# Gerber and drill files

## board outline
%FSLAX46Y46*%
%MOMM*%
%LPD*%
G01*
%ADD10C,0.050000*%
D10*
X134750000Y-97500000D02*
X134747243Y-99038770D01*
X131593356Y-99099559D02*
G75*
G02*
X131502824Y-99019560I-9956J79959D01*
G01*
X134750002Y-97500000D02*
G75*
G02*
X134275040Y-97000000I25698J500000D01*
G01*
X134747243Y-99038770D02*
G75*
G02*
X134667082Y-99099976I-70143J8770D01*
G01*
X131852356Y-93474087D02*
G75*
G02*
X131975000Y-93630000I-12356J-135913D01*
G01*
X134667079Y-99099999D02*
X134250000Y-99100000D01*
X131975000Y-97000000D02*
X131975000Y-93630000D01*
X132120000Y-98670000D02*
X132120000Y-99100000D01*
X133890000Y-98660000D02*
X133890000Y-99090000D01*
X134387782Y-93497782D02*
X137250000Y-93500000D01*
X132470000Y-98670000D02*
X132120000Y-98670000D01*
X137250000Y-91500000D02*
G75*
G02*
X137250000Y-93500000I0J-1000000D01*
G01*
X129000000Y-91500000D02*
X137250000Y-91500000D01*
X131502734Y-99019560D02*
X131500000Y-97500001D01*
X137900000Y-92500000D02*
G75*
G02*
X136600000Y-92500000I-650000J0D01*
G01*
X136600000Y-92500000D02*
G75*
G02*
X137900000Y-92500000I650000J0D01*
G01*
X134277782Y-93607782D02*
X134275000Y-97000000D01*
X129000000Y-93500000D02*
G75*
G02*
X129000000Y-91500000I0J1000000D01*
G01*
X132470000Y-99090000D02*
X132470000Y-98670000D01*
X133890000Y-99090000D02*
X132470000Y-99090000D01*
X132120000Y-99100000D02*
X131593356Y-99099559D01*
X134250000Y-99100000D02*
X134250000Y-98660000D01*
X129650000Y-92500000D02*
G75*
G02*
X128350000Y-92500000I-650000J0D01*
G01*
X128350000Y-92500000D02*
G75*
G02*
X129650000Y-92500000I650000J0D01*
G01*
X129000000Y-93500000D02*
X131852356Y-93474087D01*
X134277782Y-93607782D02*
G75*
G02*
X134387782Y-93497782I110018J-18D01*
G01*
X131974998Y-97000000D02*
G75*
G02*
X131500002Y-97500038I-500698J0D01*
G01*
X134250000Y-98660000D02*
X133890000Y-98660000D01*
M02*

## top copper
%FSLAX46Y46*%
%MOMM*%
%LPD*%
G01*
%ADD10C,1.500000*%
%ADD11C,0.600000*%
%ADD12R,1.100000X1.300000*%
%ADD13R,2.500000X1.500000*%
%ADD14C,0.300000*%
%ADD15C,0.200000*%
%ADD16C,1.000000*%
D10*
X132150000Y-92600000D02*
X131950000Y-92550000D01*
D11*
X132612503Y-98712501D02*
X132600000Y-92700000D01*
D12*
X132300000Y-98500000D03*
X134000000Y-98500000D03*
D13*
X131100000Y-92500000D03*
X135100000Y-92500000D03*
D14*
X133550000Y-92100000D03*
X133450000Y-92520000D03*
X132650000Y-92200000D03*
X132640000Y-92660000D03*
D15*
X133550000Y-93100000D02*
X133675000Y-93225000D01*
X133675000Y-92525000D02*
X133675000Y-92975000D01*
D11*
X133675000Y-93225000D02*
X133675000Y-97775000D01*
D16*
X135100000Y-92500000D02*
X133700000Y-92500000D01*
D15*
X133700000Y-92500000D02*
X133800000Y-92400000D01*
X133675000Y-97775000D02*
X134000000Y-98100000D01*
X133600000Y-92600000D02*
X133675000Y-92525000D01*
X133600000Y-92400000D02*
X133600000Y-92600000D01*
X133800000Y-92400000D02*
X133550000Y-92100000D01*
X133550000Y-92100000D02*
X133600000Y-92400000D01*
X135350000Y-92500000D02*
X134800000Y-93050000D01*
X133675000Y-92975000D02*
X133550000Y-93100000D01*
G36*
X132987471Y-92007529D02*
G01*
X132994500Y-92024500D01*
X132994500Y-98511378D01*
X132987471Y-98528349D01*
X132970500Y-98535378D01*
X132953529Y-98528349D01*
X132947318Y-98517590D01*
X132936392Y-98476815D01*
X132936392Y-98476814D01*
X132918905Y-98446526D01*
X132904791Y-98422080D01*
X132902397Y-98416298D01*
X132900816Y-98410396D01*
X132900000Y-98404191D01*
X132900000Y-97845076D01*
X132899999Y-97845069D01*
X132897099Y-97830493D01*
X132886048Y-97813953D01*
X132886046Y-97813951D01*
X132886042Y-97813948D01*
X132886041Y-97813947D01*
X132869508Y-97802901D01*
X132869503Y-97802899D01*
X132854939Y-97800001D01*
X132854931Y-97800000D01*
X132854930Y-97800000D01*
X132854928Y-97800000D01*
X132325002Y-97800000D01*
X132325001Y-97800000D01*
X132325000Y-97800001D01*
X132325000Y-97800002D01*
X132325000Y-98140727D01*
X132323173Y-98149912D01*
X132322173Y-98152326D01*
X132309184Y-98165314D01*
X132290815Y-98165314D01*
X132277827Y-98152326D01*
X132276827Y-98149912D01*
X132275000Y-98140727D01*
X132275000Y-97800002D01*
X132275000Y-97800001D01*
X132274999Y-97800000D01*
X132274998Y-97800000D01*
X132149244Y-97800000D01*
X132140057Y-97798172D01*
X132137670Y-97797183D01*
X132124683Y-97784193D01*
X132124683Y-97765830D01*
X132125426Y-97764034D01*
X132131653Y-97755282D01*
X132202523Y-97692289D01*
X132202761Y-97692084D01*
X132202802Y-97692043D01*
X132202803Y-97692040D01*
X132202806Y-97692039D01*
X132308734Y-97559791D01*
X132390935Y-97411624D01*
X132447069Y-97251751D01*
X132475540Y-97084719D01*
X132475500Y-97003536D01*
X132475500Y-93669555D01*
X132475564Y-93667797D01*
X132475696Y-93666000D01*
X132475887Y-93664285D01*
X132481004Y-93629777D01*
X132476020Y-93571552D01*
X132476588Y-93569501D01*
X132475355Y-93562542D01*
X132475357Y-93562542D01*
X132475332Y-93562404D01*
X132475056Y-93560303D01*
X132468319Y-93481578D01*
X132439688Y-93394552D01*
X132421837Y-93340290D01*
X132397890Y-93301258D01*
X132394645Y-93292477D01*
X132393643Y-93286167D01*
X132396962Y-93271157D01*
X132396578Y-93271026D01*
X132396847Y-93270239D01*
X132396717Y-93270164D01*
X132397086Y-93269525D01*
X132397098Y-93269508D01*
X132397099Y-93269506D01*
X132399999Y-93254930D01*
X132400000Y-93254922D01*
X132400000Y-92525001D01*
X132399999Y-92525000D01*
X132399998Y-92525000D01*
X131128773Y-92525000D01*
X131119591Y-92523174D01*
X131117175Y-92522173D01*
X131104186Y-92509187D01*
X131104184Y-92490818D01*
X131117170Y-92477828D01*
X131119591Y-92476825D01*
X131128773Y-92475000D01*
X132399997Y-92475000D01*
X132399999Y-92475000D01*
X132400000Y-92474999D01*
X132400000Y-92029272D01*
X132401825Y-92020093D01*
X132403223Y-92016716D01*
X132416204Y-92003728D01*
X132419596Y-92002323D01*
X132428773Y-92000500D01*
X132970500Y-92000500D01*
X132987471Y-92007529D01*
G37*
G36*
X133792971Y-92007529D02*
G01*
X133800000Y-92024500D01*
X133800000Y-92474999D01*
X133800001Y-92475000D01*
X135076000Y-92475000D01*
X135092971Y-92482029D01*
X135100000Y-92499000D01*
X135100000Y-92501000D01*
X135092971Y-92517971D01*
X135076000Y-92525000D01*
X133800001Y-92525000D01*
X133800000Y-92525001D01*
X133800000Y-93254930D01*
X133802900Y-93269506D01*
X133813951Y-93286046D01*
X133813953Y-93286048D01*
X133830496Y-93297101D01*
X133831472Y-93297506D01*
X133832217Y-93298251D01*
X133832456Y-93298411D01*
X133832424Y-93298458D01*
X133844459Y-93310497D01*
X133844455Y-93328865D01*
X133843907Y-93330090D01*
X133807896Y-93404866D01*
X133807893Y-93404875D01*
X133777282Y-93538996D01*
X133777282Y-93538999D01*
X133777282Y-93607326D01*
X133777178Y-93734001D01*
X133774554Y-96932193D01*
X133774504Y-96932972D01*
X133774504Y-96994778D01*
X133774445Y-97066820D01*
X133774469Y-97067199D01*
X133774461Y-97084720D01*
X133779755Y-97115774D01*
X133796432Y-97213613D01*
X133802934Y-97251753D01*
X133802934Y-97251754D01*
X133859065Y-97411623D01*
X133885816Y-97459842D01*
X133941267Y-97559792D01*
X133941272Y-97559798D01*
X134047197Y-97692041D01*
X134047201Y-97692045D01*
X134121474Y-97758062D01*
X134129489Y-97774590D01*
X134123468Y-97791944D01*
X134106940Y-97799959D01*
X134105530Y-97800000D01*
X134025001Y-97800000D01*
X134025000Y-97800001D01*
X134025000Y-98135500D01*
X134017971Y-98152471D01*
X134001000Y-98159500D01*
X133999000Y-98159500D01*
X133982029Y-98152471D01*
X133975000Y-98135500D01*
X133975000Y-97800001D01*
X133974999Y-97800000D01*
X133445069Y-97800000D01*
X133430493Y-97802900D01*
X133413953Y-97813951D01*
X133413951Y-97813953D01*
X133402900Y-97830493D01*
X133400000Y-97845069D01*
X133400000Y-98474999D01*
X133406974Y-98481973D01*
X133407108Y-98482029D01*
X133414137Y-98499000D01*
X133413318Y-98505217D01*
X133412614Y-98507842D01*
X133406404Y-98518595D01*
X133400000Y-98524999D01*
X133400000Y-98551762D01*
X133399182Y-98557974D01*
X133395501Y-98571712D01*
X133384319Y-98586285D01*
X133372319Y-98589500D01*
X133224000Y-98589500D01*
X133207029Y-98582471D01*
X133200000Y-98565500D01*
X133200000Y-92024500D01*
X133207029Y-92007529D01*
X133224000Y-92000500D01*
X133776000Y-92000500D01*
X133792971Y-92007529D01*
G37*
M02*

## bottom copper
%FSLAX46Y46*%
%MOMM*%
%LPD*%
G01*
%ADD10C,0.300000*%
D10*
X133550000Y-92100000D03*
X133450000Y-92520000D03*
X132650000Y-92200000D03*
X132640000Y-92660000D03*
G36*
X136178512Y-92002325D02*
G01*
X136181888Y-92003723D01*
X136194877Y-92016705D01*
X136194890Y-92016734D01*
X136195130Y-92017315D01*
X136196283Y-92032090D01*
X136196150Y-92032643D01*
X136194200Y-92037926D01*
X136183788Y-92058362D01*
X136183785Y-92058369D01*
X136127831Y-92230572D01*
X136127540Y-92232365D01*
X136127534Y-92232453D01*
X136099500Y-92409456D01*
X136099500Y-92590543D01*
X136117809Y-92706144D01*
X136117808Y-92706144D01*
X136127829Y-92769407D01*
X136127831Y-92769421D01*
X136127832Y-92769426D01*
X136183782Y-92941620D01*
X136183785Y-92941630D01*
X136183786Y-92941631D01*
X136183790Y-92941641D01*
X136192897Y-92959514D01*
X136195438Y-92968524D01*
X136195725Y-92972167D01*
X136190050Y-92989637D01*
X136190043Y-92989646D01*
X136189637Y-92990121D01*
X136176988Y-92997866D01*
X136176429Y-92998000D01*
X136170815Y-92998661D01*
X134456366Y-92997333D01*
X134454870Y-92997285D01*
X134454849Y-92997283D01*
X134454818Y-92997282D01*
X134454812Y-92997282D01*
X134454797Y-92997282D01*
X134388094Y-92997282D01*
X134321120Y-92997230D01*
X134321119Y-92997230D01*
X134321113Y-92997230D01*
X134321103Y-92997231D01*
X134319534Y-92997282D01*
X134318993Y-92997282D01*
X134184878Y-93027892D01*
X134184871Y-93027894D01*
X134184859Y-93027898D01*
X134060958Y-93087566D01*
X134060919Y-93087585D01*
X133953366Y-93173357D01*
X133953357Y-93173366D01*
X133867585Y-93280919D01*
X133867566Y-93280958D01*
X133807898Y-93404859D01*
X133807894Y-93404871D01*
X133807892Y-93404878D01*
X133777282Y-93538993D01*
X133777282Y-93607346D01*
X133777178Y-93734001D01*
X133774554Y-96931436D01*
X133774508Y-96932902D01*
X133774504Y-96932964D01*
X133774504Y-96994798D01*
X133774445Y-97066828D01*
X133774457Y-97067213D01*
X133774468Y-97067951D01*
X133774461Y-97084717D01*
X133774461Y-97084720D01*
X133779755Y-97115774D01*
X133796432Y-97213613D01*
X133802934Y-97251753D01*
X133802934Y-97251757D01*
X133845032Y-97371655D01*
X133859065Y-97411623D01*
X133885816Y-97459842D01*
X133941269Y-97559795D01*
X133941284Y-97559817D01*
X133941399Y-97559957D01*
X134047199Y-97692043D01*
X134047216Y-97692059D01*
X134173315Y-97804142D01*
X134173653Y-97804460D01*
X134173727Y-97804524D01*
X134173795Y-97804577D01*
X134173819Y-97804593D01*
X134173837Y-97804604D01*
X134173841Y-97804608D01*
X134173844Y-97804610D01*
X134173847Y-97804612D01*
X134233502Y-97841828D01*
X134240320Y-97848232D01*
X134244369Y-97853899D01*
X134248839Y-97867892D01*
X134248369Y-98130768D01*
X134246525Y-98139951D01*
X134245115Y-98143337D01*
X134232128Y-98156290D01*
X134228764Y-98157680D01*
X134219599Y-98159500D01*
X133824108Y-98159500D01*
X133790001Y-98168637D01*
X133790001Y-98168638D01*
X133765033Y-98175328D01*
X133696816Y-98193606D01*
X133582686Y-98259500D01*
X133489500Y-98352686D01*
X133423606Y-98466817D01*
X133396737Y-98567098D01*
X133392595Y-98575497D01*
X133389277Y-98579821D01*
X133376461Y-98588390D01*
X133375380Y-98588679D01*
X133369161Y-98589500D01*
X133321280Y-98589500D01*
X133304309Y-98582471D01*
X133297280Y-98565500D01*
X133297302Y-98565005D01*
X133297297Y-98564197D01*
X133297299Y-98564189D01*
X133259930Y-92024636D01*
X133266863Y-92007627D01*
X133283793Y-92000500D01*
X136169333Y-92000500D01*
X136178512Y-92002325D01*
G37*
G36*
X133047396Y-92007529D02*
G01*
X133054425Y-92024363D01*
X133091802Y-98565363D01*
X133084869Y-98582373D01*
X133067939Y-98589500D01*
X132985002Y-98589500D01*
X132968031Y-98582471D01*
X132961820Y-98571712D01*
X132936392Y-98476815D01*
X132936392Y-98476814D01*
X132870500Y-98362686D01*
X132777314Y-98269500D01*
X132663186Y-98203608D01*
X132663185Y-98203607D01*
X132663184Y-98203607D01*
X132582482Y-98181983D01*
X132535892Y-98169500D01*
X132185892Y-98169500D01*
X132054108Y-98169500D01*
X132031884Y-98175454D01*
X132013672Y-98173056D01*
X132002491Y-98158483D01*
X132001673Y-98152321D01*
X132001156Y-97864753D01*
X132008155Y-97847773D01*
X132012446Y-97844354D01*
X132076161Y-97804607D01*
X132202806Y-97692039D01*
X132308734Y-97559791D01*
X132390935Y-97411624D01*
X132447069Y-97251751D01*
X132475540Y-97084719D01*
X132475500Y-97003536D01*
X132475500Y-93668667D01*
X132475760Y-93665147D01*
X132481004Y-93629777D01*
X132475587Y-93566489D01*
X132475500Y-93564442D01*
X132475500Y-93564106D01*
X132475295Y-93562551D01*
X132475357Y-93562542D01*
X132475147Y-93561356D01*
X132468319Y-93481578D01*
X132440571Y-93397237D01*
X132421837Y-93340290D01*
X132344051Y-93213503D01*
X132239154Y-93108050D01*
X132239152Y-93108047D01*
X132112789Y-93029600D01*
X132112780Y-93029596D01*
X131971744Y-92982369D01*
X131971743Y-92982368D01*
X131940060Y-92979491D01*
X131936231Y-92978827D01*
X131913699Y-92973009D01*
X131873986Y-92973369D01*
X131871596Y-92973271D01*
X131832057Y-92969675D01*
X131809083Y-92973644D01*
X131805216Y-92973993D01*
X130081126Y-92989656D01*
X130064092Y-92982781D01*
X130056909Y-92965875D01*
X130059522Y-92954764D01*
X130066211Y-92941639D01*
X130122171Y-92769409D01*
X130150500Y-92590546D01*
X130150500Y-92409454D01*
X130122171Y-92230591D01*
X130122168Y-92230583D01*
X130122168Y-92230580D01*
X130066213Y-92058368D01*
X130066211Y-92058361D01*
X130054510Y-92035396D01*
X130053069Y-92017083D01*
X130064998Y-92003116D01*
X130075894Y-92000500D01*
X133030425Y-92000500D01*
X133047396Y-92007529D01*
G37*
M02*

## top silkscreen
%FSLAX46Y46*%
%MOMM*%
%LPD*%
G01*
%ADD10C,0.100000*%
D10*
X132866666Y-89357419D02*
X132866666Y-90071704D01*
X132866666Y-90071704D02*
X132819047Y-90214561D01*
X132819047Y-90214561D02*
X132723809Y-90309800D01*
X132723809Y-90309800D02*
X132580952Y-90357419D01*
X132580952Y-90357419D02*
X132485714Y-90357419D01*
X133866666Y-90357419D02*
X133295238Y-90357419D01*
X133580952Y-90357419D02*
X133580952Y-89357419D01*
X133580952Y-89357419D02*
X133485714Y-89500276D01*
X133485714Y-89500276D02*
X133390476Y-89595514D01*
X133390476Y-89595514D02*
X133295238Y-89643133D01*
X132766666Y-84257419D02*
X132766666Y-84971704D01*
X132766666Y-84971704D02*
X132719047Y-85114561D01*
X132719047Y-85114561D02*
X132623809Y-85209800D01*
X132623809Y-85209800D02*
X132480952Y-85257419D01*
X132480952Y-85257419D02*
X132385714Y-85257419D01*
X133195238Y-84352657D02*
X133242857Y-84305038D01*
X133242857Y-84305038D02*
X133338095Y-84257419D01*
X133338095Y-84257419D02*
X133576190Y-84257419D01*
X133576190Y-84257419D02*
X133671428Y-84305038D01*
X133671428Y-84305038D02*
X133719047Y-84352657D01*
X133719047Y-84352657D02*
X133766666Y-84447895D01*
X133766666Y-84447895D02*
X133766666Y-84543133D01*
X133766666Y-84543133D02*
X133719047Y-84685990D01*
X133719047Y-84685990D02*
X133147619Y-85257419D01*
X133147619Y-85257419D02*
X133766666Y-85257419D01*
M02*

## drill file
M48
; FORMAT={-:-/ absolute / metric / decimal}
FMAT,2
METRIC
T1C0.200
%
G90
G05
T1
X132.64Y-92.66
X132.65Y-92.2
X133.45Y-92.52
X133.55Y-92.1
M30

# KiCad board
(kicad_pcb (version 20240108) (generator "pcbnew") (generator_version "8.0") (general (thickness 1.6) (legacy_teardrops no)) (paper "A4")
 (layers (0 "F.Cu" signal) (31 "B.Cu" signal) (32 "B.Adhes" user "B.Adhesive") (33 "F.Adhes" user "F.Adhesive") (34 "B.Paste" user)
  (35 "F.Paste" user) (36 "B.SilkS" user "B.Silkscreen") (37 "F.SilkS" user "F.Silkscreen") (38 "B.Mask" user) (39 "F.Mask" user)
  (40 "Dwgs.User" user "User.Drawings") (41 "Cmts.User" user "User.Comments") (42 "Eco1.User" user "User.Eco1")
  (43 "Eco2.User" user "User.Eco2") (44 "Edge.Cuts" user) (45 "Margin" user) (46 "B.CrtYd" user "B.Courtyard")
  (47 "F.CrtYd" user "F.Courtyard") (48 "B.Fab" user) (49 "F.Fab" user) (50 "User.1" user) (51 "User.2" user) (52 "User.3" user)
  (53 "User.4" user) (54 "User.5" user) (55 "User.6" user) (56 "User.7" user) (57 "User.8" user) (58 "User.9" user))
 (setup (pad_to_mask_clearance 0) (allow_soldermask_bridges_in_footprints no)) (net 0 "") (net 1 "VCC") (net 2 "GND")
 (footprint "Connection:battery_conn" (layer "F.Cu") (at 133.2 98.5)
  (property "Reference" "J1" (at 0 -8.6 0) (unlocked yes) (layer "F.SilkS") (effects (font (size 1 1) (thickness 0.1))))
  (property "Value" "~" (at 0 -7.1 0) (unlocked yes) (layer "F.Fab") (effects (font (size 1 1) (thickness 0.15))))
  (pad "1" smd rect (at -0.9 0) (size 1.1 1.3) (layers "F.Cu" "F.Paste" "F.Mask") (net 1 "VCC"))
  (pad "2" smd rect (at 0.8 0) (size 1.1 1.3) (layers "F.Cu" "F.Paste" "F.Mask") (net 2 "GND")))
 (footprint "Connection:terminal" (layer "F.Cu") (at 133.1 94.5)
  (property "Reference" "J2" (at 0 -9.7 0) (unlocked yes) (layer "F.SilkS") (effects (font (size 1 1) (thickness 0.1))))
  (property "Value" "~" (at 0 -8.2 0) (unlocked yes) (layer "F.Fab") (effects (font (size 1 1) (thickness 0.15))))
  (pad "1" smd rect (at -2 -2) (size 2.5 1.5) (layers "F.Cu" "F.Paste" "F.Mask") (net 1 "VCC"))
  (pad "2" smd rect (at 2 -2) (size 2.5 1.5) (layers "F.Cu" "F.Paste" "F.Mask") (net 2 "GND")))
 (gr_line (start 132.15 92.6) (end 131.95 92.55) (stroke (width 1.5) (type default)) (layer "F.Cu") (net 1))
 (gr_line (start 132.612503 98.712501) (end 132.6 92.7) (stroke (width 0.6) (type default)) (layer "F.Cu") (net 1))
 (gr_line (start 134.75 97.5) (end 134.747243 99.03877) (stroke (width 0.05) (type default)) (layer "Edge.Cuts"))
 (gr_arc (start 131.593356 99.099559) (mid 131.53 99.08) (end 131.502734 99.01956) (stroke (width 0.05) (type default)) (layer "Edge.Cuts"))
 (gr_arc (start 134.750002 97.5) (mid 134.412683 97.344828) (end 134.275004 97) (stroke (width 0.05) (type default)) (layer "Edge.Cuts"))
 (gr_arc (start 134.747243 99.03877) (mid 134.72 99.086194) (end 134.667079 99.099999) (stroke (width 0.05) (type default))
  (layer "Edge.Cuts"))
 (gr_arc (start 131.852356 93.474087) (mid 131.947264 93.525624) (end 131.975 93.63) (stroke (width 0.05) (type default))
  (layer "Edge.Cuts"))
 (gr_line (start 134.667079 99.099999) (end 134.25 99.1) (stroke (width 0.05) (type default)) (layer "Edge.Cuts"))
 (gr_line (start 131.975 97) (end 131.975 93.63) (stroke (width 0.05) (type default)) (layer "Edge.Cuts"))
 (gr_line (start 132.12 98.67) (end 132.12 99.1) (stroke (width 0.05) (type default)) (layer "Edge.Cuts"))
 (gr_line (start 133.89 98.66) (end 133.89 99.09) (stroke (width 0.05) (type default)) (layer "Edge.Cuts"))
 (gr_line (start 134.387782 93.497782) (end 137.25 93.5) (stroke (width 0.05) (type default)) (layer "Edge.Cuts"))
 (gr_line (start 132.47 98.67) (end 132.12 98.67) (stroke (width 0.05) (type default)) (layer "Edge.Cuts"))
 (gr_arc (start 137.25 91.5) (mid 138.25 92.5) (end 137.25 93.5) (stroke (width 0.05) (type default)) (layer "Edge.Cuts"))
 (gr_line (start 129 91.5) (end 137.25 91.5) (stroke (width 0.05) (type default)) (layer "Edge.Cuts"))
 (gr_line (start 131.502734 99.01956) (end 131.5 97.500001) (stroke (width 0.05) (type default)) (layer "Edge.Cuts"))
 (gr_circle (center 137.25 92.5) (end 137.9 92.5) (stroke (width 0.05) (type default)) (fill none) (layer "Edge.Cuts"))
 (gr_line (start 134.277782 93.607782) (end 134.275 97) (stroke (width 0.05) (type default)) (layer "Edge.Cuts"))
 (gr_arc (start 129 93.5) (mid 128 92.5) (end 129 91.5) (stroke (width 0.05) (type default)) (layer "Edge.Cuts"))
 (gr_line (start 132.47 99.09) (end 132.47 98.67) (stroke (width 0.05) (type default)) (layer "Edge.Cuts"))
 (gr_line (start 133.89 99.09) (end 132.47 99.09) (stroke (width 0.05) (type default)) (layer "Edge.Cuts"))
 (gr_line (start 132.12 99.1) (end 131.593356 99.099559) (stroke (width 0.05) (type default)) (layer "Edge.Cuts"))
 (gr_line (start 134.25 99.1) (end 134.25 98.66) (stroke (width 0.05) (type default)) (layer "Edge.Cuts"))
 (gr_circle (center 129 92.5) (end 129.65 92.5) (stroke (width 0.05) (type default)) (fill none) (layer "Edge.Cuts"))
 (gr_line (start 129 93.5) (end 131.852356 93.474087) (stroke (width 0.05) (type default)) (layer "Edge.Cuts"))
 (gr_arc (start 134.277782 93.607782) (mid 134.31 93.53) (end 134.387782 93.497782) (stroke (width 0.05) (type default)) (layer "Edge.Cuts"))
 (gr_arc (start 131.974998 97) (mid 131.837318 97.344828) (end 131.5 97.500001) (stroke (width 0.05) (type default)) (layer "Edge.Cuts"))
 (gr_line (start 134.25 98.66) (end 133.89 98.66) (stroke (width 0.05) (type default)) (layer "Edge.Cuts"))
 (segment (start 133.55 93.1) (end 133.675 93.225) (width 0.2) (layer "F.Cu") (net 2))
 (segment (start 133.675 92.525) (end 133.675 92.975) (width 0.2) (layer "F.Cu") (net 2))
 (segment (start 133.675 93.225) (end 133.675 97.775) (width 0.6) (layer "F.Cu") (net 2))
 (segment (start 135.1 92.5) (end 133.7 92.5) (width 1) (layer "F.Cu") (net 2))
 (segment (start 133.7 92.5) (end 133.8 92.4) (width 0.2) (layer "F.Cu") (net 2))
 (segment (start 133.675 97.775) (end 134 98.1) (width 0.2) (layer "F.Cu") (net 2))
 (segment (start 133.6 92.6) (end 133.675 92.525) (width 0.2) (layer "F.Cu") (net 2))
 (segment (start 133.6 92.4) (end 133.6 92.6) (width 0.2) (layer "F.Cu") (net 2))
 (segment (start 133.8 92.4) (end 133.55 92.1) (width 0.2) (layer "F.Cu") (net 2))
 (segment (start 133.55 92.1) (end 133.6 92.4) (width 0.2) (layer "F.Cu") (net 2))
 (segment (start 135.35 92.5) (end 134.8 93.05) (width 0.2) (layer "F.Cu") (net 2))
 (segment (start 133.675 92.975) (end 133.55 93.1) (width 0.2) (layer "F.Cu") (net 2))
 (via (at 133.55 92.1) (size 0.3) (drill 0.2) (layers "F.Cu" "B.Cu") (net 2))
 (via (at 133.45 92.52) (size 0.3) (drill 0.2) (layers "F.Cu" "B.Cu") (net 2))
 (via (at 132.65 92.2) (size 0.3) (drill 0.2) (layers "F.Cu" "B.Cu") (free yes) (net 1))
 (via (at 132.64 92.66) (size 0.3) (drill 0.2) (layers "F.Cu" "B.Cu") (free yes) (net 1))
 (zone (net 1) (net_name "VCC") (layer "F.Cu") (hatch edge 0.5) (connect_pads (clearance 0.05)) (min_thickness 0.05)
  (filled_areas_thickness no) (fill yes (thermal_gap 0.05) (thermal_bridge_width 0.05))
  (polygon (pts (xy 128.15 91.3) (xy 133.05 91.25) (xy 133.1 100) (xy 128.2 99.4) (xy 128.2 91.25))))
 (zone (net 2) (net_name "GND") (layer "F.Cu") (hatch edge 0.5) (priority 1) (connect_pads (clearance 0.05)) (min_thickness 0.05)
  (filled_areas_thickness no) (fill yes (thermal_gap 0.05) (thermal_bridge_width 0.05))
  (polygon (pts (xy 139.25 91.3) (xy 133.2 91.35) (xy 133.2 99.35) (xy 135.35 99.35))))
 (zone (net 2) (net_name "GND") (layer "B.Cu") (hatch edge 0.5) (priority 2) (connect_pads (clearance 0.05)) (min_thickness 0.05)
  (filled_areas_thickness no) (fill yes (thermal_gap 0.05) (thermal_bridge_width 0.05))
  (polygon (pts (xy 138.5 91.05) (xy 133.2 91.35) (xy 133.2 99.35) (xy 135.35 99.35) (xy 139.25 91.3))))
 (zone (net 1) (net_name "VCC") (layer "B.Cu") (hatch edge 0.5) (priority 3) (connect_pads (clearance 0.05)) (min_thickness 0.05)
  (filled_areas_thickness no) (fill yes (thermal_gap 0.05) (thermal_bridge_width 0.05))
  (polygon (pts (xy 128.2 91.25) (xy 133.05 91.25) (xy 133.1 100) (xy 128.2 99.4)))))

